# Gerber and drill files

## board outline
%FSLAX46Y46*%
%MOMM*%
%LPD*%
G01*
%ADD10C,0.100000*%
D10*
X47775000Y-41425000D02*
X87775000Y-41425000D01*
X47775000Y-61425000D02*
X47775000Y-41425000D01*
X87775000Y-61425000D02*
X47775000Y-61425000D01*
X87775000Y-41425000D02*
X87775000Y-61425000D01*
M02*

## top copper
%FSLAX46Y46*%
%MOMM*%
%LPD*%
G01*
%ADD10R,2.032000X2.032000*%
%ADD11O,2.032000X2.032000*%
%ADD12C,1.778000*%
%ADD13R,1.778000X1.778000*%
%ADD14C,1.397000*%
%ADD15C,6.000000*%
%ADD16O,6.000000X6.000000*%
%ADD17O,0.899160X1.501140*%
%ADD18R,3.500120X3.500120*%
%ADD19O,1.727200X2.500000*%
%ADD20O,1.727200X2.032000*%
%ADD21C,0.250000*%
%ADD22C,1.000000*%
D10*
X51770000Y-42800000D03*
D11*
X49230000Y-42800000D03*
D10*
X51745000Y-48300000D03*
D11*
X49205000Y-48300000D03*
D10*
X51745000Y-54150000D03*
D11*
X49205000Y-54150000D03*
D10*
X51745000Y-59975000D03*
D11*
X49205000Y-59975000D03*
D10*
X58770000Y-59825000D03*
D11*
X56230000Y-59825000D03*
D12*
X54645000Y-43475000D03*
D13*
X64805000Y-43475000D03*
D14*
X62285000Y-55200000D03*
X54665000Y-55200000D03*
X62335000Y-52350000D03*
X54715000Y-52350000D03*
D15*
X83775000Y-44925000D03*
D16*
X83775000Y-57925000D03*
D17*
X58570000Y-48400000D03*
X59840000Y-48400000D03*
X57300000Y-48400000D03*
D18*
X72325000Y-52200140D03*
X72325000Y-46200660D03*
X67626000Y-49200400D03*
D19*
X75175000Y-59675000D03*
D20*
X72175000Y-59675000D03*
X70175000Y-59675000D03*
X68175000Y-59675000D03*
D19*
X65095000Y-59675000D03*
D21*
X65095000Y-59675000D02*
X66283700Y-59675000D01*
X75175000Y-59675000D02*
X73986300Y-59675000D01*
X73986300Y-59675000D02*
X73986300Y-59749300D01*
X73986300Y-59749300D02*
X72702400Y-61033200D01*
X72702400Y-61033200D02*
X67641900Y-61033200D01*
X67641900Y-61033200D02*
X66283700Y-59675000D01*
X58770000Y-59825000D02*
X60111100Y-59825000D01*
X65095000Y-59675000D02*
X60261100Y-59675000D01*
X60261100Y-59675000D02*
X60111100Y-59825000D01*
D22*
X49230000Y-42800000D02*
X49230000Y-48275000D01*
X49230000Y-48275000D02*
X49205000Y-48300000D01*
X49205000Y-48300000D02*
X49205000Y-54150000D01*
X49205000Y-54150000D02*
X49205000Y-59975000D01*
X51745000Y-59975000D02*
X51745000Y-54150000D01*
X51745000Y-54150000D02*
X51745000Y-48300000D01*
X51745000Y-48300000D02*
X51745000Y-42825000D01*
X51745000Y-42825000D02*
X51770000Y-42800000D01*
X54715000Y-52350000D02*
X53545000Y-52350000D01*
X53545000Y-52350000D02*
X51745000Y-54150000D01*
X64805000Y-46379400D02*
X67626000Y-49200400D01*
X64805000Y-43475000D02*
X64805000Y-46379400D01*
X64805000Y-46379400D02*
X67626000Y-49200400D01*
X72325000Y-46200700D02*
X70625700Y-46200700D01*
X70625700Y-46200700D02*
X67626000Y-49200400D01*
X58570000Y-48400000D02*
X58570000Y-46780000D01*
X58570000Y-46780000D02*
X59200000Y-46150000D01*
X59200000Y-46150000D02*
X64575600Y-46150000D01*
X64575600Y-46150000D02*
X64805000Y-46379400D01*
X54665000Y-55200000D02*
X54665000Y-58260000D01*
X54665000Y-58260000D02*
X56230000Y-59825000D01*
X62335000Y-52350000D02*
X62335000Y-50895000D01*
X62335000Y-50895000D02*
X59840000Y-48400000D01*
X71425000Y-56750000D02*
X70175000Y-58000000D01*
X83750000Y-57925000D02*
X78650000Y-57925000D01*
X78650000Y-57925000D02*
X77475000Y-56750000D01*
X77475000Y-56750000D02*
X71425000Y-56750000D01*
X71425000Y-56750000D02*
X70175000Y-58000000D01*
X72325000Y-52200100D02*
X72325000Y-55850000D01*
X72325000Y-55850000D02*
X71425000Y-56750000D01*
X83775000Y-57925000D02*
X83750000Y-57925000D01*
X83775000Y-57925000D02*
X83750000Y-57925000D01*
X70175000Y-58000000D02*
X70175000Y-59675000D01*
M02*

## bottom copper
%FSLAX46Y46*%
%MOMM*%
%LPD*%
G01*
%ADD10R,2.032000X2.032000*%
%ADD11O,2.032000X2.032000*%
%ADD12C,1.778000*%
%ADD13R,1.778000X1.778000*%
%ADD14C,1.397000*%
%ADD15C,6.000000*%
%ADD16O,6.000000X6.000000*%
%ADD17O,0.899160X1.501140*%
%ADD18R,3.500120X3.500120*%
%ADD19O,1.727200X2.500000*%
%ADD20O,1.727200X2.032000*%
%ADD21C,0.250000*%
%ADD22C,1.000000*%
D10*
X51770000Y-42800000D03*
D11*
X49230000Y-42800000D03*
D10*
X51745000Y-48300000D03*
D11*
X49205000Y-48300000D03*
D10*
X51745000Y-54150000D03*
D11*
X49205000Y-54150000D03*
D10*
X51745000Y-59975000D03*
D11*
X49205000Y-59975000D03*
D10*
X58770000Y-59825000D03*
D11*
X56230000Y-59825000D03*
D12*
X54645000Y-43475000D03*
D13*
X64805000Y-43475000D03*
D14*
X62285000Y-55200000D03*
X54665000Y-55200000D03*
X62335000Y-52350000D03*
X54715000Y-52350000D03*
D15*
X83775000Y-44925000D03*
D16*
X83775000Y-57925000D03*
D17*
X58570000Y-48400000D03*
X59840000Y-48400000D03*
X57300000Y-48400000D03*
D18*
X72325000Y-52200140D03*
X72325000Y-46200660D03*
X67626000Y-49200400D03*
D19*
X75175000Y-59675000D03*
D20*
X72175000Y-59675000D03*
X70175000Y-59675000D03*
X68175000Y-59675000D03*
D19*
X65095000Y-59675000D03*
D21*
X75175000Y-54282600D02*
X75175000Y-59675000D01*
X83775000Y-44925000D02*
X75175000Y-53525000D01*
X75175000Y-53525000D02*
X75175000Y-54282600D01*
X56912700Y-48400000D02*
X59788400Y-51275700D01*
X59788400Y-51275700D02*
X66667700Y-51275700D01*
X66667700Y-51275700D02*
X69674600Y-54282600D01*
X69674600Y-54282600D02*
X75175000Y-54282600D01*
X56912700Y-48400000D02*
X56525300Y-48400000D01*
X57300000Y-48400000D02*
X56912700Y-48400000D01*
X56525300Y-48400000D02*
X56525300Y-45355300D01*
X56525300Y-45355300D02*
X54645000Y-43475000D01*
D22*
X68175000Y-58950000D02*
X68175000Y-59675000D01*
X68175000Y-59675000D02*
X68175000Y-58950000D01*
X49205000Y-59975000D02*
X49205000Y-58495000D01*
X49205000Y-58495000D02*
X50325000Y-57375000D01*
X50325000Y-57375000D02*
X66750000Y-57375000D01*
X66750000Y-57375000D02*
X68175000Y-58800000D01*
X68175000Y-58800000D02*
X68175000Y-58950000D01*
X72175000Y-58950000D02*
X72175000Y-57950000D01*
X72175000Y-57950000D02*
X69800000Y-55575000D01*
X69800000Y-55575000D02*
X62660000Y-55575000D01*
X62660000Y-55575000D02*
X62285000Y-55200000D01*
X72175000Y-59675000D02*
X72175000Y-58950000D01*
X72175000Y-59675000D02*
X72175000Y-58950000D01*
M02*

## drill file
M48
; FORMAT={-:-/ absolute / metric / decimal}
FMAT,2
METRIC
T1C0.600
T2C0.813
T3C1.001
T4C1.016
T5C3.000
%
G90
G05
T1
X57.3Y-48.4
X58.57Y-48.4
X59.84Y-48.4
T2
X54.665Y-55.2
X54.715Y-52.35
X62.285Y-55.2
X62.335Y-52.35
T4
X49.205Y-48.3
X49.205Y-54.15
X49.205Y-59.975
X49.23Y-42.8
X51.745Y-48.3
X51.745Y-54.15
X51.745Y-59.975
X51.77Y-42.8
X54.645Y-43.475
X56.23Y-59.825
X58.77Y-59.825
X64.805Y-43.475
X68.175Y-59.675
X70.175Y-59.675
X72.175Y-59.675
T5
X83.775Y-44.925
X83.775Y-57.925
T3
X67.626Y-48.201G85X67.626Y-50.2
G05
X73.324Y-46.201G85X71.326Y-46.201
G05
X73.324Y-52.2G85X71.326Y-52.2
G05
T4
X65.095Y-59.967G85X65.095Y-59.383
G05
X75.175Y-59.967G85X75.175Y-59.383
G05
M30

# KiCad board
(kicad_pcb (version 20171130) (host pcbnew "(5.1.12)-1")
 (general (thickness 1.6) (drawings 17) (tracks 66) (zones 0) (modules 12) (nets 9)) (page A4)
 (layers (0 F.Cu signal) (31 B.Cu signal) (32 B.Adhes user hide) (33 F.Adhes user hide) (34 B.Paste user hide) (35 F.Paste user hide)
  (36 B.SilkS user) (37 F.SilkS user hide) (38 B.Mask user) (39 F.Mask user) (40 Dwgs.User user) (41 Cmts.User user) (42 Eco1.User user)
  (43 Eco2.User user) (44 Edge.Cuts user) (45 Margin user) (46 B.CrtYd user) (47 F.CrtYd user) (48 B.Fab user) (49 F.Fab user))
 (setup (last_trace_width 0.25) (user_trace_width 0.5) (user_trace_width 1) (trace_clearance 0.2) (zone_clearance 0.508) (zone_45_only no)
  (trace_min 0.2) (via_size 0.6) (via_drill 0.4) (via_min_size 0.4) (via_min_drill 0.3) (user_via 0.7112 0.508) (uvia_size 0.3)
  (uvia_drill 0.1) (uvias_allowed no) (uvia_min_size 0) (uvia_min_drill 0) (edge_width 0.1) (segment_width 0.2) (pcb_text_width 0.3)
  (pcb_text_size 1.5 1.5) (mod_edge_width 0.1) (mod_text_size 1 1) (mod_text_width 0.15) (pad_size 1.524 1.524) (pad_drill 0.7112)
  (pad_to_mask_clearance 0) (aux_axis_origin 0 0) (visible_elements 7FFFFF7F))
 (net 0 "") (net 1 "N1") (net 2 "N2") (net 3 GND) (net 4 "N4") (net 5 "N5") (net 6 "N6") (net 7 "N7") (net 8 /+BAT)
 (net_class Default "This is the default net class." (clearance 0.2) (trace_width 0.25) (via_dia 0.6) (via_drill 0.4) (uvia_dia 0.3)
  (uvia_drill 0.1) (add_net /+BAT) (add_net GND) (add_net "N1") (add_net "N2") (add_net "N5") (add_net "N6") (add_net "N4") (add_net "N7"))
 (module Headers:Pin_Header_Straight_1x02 (layer F.Cu) (at 50.5 42.8 180)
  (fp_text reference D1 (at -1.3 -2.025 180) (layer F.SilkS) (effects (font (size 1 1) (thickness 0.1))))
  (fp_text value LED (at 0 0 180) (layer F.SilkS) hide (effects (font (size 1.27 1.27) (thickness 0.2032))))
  (pad 1 thru_hole rect (at -1.27 0 180) (size 2.032 2.032) (drill 1.016) (layers *.Cu *.Mask F.SilkS) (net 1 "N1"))
  (pad 2 thru_hole oval (at 1.27 0 180) (size 2.032 2.032) (drill 1.016) (layers *.Cu *.Mask F.SilkS) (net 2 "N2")))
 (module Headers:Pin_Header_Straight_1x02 (layer F.Cu) (at 50.475 48.3 180)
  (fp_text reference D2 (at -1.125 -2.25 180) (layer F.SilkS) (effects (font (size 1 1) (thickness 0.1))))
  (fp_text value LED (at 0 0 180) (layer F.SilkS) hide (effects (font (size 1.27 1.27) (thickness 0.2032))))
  (pad 1 thru_hole rect (at -1.27 0 180) (size 2.032 2.032) (drill 1.016) (layers *.Cu *.Mask F.SilkS) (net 1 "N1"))
  (pad 2 thru_hole oval (at 1.27 0 180) (size 2.032 2.032) (drill 1.016) (layers *.Cu *.Mask F.SilkS) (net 2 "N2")))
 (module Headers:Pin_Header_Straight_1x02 (layer F.Cu) (at 50.475 54.15 180)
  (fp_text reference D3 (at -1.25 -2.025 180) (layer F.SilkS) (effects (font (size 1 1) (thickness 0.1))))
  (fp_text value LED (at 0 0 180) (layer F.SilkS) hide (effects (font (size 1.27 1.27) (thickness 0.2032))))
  (pad 1 thru_hole rect (at -1.27 0 180) (size 2.032 2.032) (drill 1.016) (layers *.Cu *.Mask F.SilkS) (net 1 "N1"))
  (pad 2 thru_hole oval (at 1.27 0 180) (size 2.032 2.032) (drill 1.016) (layers *.Cu *.Mask F.SilkS) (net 2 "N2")))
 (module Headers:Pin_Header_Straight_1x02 (layer F.Cu) (at 50.475 59.975 180)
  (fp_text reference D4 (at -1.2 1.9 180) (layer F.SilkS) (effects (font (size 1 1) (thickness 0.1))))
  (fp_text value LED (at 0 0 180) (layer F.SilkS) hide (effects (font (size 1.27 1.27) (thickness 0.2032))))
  (pad 1 thru_hole rect (at -1.27 0 180) (size 2.032 2.032) (drill 1.016) (layers *.Cu *.Mask F.SilkS) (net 1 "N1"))
  (pad 2 thru_hole oval (at 1.27 0 180) (size 2.032 2.032) (drill 1.016) (layers *.Cu *.Mask F.SilkS) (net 2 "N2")))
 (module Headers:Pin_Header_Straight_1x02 (layer F.Cu) (at 57.5 59.825 180)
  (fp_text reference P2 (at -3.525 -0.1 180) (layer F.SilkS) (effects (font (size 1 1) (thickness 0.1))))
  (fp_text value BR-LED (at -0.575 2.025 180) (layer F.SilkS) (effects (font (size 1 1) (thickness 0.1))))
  (pad 1 thru_hole rect (at -1.27 0 180) (size 2.032 2.032) (drill 1.016) (layers *.Cu *.Mask F.SilkS) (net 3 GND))
  (pad 2 thru_hole oval (at 1.27 0 180) (size 2.032 2.032) (drill 1.016) (layers *.Cu *.Mask F.SilkS) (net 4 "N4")))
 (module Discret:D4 (layer F.Cu) (at 59.725 43.475)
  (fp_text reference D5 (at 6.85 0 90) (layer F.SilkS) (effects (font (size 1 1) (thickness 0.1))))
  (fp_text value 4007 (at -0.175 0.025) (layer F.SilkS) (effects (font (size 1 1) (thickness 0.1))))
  (pad 2 thru_hole circle (at -5.08 0) (size 1.778 1.778) (drill 1.016) (layers *.Cu *.Mask F.SilkS) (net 3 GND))
  (pad 1 thru_hole rect (at 5.08 0) (size 1.778 1.778) (drill 1.016) (layers *.Cu *.Mask F.SilkS) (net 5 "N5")))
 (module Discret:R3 (layer F.Cu) (at 58.475 55.2 180)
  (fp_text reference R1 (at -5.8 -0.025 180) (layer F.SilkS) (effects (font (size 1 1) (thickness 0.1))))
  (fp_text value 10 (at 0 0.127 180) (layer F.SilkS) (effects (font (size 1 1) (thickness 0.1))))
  (pad 1 thru_hole circle (at -3.81 0 180) (size 1.397 1.397) (drill 0.8128) (layers *.Cu *.Mask F.SilkS) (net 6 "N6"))
  (pad 2 thru_hole circle (at 3.81 0 180) (size 1.397 1.397) (drill 0.8128) (layers *.Cu *.Mask F.SilkS) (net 4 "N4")))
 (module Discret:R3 (layer F.Cu) (at 58.525 52.35 180)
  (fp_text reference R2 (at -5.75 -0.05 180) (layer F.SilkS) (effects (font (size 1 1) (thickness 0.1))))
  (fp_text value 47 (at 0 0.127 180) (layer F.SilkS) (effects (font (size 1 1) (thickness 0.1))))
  (pad 1 thru_hole circle (at -3.81 0 180) (size 1.397 1.397) (drill 0.8128) (layers *.Cu *.Mask F.SilkS) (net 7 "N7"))
  (pad 2 thru_hole circle (at 3.81 0 180) (size 1.397 1.397) (drill 0.8128) (layers *.Cu *.Mask F.SilkS) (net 1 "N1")))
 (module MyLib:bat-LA (layer F.Cu) (at 83.775 51.425 270)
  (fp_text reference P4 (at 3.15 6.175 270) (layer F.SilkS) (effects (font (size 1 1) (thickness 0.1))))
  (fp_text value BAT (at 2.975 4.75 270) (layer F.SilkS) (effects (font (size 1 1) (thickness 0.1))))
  (pad 1 thru_hole circle (at -6.5 0 270) (size 6 6) (drill 3) (layers *.Cu *.Mask F.SilkS) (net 3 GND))
  (pad 2 thru_hole oval (at 6.5 0 270) (size 6 6) (drill 3) (layers *.Cu *.Mask F.SilkS) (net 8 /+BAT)))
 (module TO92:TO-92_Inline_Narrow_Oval (layer F.Cu) (at 57.3 48.4)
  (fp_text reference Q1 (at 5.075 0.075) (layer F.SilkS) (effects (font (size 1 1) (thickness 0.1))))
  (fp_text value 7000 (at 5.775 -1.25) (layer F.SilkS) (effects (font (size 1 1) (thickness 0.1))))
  (pad 2 thru_hole oval (at 1.27 0 180) (size 0.89916 1.50114) (drill 0.6) (layers *.Cu *.Mask F.SilkS) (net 5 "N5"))
  (pad 3 thru_hole oval (at 2.54 0 180) (size 0.89916 1.50114) (drill 0.6) (layers *.Cu *.Mask F.SilkS) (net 7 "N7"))
  (pad 1 thru_hole oval (at 0 0 180) (size 0.89916 1.50114) (drill 0.6) (layers *.Cu *.Mask F.SilkS) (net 3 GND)))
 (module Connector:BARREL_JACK (layer F.Cu) (at 72.325 46 270)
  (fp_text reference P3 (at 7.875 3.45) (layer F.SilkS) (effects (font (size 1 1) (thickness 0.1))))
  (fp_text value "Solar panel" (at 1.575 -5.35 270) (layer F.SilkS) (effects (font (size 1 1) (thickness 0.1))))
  (pad 1 thru_hole rect (at 6.20014 0 270) (size 3.50012 3.50012) (drill oval 1.00076 2.99974) (layers *.Cu *.Mask F.SilkS) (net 8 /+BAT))
  (pad 2 thru_hole rect (at 0.20066 0 270) (size 3.50012 3.50012) (drill oval 1.00076 2.99974) (layers *.Cu *.Mask F.SilkS) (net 5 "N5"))
  (pad 3 thru_hole rect (at 3.2004 4.699 270) (size 3.50012 3.50012) (drill oval 2.99974 1.00076) (layers *.Cu *.Mask F.SilkS) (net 5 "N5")))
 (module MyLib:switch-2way (layer F.Cu) (at 70.175 59.675 180)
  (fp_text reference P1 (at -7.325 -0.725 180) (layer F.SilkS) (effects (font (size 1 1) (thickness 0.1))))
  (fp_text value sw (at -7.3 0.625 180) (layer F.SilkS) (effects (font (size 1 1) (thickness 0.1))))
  (pad 1 thru_hole oval (at -5 0 180) (size 1.7272 2.5) (drill oval 1.016 1.6) (layers *.Cu *.Mask F.SilkS) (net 3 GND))
  (pad 2 thru_hole oval (at -2 0 180) (size 1.7272 2.032) (drill 1.016) (layers *.Cu *.Mask F.SilkS) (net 6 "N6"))
  (pad 3 thru_hole oval (at 0 0 180) (size 1.7272 2.032) (drill 1.016) (layers *.Cu *.Mask F.SilkS) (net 8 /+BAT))
  (pad 4 thru_hole oval (at 2 0 180) (size 1.7272 2.032) (drill 1.016) (layers *.Cu *.Mask F.SilkS) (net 2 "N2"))
  (pad 5 thru_hole oval (at 5.08 0 180) (size 1.7272 2.5) (drill oval 1.016 1.6) (layers *.Cu *.Mask F.SilkS) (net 3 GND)))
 (gr_line (start 47.775 41.425) (end 87.775 41.425) (angle 90) (layer Edge.Cuts) (width 0.1))
 (gr_line (start 47.775 61.425) (end 47.775 41.425) (angle 90) (layer Edge.Cuts) (width 0.1))
 (gr_line (start 87.775 61.425) (end 47.775 61.425) (angle 90) (layer Edge.Cuts) (width 0.1))
 (gr_line (start 87.775 41.425) (end 87.775 61.425) (angle 90) (layer Edge.Cuts) (width 0.1))
 (segment (start 75.175 54.2826) (end 75.175 59.675) (width 0.25) (layer B.Cu) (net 3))
 (segment (start 83.775 44.925) (end 75.175 53.525) (width 0.25) (layer B.Cu) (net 3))
 (segment (start 75.175 53.525) (end 75.175 54.2826) (width 0.25) (layer B.Cu) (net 3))
 (segment (start 56.9127 48.4) (end 59.7884 51.2757) (width 0.25) (layer B.Cu) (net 3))
 (segment (start 59.7884 51.2757) (end 66.6677 51.2757) (width 0.25) (layer B.Cu) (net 3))
 (segment (start 66.6677 51.2757) (end 69.6746 54.2826) (width 0.25) (layer B.Cu) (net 3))
 (segment (start 69.6746 54.2826) (end 75.175 54.2826) (width 0.25) (layer B.Cu) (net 3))
 (segment (start 56.9127 48.4) (end 56.5253 48.4) (width 0.25) (layer B.Cu) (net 3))
 (segment (start 57.3 48.4) (end 56.9127 48.4) (width 0.25) (layer B.Cu) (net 3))
 (segment (start 56.5253 48.4) (end 56.5253 45.3553) (width 0.25) (layer B.Cu) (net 3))
 (segment (start 56.5253 45.3553) (end 54.645 43.475) (width 0.25) (layer B.Cu) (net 3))
 (segment (start 65.095 59.675) (end 66.2837 59.675) (width 0.25) (layer F.Cu) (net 3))
 (segment (start 75.175 59.675) (end 73.9863 59.675) (width 0.25) (layer F.Cu) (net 3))
 (segment (start 73.9863 59.675) (end 73.9863 59.7493) (width 0.25) (layer F.Cu) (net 3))
 (segment (start 73.9863 59.7493) (end 72.7024 61.0332) (width 0.25) (layer F.Cu) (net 3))
 (segment (start 72.7024 61.0332) (end 67.6419 61.0332) (width 0.25) (layer F.Cu) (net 3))
 (segment (start 67.6419 61.0332) (end 66.2837 59.675) (width 0.25) (layer F.Cu) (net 3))
 (segment (start 58.77 59.825) (end 60.1111 59.825) (width 0.25) (layer F.Cu) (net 3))
 (segment (start 65.095 59.675) (end 60.2611 59.675) (width 0.25) (layer F.Cu) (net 3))
 (segment (start 60.2611 59.675) (end 60.1111 59.825) (width 0.25) (layer F.Cu) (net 3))
 (segment (start 68.175 58.95) (end 68.175 59.675) (width 1) (layer B.Cu) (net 2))
 (segment (start 68.175 59.675) (end 68.175 58.95) (width 1) (layer B.Cu) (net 2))
 (segment (start 49.23 42.8) (end 49.23 48.275) (width 1) (layer F.Cu) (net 2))
 (segment (start 49.23 48.275) (end 49.205 48.3) (width 1) (layer F.Cu) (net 2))
 (segment (start 49.205 48.3) (end 49.205 54.15) (width 1) (layer F.Cu) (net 2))
 (segment (start 49.205 54.15) (end 49.205 59.975) (width 1) (layer F.Cu) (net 2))
 (segment (start 49.205 59.975) (end 49.205 58.495) (width 1) (layer B.Cu) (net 2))
 (segment (start 49.205 58.495) (end 50.325 57.375) (width 1) (layer B.Cu) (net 2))
 (segment (start 50.325 57.375) (end 66.75 57.375) (width 1) (layer B.Cu) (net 2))
 (segment (start 66.75 57.375) (end 68.175 58.8) (width 1) (layer B.Cu) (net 2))
 (segment (start 68.175 58.8) (end 68.175 58.95) (width 1) (layer B.Cu) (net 2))
 (segment (start 51.745 59.975) (end 51.745 54.15) (width 1) (layer F.Cu) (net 1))
 (segment (start 51.745 54.15) (end 51.745 48.3) (width 1) (layer F.Cu) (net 1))
 (segment (start 51.745 48.3) (end 51.745 42.825) (width 1) (layer F.Cu) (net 1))
 (segment (start 51.745 42.825) (end 51.77 42.8) (width 1) (layer F.Cu) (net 1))
 (segment (start 54.715 52.35) (end 53.545 52.35) (width 1) (layer F.Cu) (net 1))
 (segment (start 53.545 52.35) (end 51.745 54.15) (width 1) (layer F.Cu) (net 1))
 (segment (start 64.805 46.3794) (end 67.626 49.2004) (width 1) (layer F.Cu) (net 5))
 (segment (start 64.805 43.475) (end 64.805 46.3794) (width 1) (layer F.Cu) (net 5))
 (segment (start 64.805 46.3794) (end 67.626 49.2004) (width 1) (layer F.Cu) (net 5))
 (segment (start 72.325 46.2007) (end 70.6257 46.2007) (width 1) (layer F.Cu) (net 5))
 (segment (start 70.6257 46.2007) (end 67.626 49.2004) (width 1) (layer F.Cu) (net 5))
 (segment (start 58.57 48.4) (end 58.57 46.78) (width 1) (layer F.Cu) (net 5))
 (segment (start 58.57 46.78) (end 59.2 46.15) (width 1) (layer F.Cu) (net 5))
 (segment (start 59.2 46.15) (end 64.5756 46.15) (width 1) (layer F.Cu) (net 5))
 (segment (start 64.5756 46.15) (end 64.805 46.3794) (width 1) (layer F.Cu) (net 5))
 (segment (start 72.175 58.95) (end 72.175 57.95) (width 1) (layer B.Cu) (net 6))
 (segment (start 72.175 57.95) (end 69.8 55.575) (width 1) (layer B.Cu) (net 6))
 (segment (start 69.8 55.575) (end 62.66 55.575) (width 1) (layer B.Cu) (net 6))
 (segment (start 62.66 55.575) (end 62.285 55.2) (width 1) (layer B.Cu) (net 6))
 (segment (start 72.175 59.675) (end 72.175 58.95) (width 1) (layer B.Cu) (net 6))
 (segment (start 72.175 59.675) (end 72.175 58.95) (width 1) (layer B.Cu) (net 6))
 (segment (start 54.665 55.2) (end 54.665 58.26) (width 1) (layer F.Cu) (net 4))
 (segment (start 54.665 58.26) (end 56.23 59.825) (width 1) (layer F.Cu) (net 4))
 (segment (start 62.335 52.35) (end 62.335 50.895) (width 1) (layer F.Cu) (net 7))
 (segment (start 62.335 50.895) (end 59.84 48.4) (width 1) (layer F.Cu) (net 7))
 (segment (start 71.425 56.75) (end 70.175 58) (width 1) (layer F.Cu) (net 8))
 (segment (start 83.75 57.925) (end 78.65 57.925) (width 1) (layer F.Cu) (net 8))
 (segment (start 78.65 57.925) (end 77.475 56.75) (width 1) (layer F.Cu) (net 8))
 (segment (start 77.475 56.75) (end 71.425 56.75) (width 1) (layer F.Cu) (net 8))
 (segment (start 71.425 56.75) (end 70.175 58) (width 1) (layer F.Cu) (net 8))
 (segment (start 72.325 52.2001) (end 72.325 55.85) (width 1) (layer F.Cu) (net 8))
 (segment (start 72.325 55.85) (end 71.425 56.75) (width 1) (layer F.Cu) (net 8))
 (segment (start 83.775 57.925) (end 83.75 57.925) (width 1) (layer F.Cu) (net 8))
 (segment (start 83.775 57.925) (end 83.75 57.925) (width 1) (layer F.Cu) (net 8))
 (segment (start 70.175 58) (end 70.175 59.675) (width 1) (layer F.Cu) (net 8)))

